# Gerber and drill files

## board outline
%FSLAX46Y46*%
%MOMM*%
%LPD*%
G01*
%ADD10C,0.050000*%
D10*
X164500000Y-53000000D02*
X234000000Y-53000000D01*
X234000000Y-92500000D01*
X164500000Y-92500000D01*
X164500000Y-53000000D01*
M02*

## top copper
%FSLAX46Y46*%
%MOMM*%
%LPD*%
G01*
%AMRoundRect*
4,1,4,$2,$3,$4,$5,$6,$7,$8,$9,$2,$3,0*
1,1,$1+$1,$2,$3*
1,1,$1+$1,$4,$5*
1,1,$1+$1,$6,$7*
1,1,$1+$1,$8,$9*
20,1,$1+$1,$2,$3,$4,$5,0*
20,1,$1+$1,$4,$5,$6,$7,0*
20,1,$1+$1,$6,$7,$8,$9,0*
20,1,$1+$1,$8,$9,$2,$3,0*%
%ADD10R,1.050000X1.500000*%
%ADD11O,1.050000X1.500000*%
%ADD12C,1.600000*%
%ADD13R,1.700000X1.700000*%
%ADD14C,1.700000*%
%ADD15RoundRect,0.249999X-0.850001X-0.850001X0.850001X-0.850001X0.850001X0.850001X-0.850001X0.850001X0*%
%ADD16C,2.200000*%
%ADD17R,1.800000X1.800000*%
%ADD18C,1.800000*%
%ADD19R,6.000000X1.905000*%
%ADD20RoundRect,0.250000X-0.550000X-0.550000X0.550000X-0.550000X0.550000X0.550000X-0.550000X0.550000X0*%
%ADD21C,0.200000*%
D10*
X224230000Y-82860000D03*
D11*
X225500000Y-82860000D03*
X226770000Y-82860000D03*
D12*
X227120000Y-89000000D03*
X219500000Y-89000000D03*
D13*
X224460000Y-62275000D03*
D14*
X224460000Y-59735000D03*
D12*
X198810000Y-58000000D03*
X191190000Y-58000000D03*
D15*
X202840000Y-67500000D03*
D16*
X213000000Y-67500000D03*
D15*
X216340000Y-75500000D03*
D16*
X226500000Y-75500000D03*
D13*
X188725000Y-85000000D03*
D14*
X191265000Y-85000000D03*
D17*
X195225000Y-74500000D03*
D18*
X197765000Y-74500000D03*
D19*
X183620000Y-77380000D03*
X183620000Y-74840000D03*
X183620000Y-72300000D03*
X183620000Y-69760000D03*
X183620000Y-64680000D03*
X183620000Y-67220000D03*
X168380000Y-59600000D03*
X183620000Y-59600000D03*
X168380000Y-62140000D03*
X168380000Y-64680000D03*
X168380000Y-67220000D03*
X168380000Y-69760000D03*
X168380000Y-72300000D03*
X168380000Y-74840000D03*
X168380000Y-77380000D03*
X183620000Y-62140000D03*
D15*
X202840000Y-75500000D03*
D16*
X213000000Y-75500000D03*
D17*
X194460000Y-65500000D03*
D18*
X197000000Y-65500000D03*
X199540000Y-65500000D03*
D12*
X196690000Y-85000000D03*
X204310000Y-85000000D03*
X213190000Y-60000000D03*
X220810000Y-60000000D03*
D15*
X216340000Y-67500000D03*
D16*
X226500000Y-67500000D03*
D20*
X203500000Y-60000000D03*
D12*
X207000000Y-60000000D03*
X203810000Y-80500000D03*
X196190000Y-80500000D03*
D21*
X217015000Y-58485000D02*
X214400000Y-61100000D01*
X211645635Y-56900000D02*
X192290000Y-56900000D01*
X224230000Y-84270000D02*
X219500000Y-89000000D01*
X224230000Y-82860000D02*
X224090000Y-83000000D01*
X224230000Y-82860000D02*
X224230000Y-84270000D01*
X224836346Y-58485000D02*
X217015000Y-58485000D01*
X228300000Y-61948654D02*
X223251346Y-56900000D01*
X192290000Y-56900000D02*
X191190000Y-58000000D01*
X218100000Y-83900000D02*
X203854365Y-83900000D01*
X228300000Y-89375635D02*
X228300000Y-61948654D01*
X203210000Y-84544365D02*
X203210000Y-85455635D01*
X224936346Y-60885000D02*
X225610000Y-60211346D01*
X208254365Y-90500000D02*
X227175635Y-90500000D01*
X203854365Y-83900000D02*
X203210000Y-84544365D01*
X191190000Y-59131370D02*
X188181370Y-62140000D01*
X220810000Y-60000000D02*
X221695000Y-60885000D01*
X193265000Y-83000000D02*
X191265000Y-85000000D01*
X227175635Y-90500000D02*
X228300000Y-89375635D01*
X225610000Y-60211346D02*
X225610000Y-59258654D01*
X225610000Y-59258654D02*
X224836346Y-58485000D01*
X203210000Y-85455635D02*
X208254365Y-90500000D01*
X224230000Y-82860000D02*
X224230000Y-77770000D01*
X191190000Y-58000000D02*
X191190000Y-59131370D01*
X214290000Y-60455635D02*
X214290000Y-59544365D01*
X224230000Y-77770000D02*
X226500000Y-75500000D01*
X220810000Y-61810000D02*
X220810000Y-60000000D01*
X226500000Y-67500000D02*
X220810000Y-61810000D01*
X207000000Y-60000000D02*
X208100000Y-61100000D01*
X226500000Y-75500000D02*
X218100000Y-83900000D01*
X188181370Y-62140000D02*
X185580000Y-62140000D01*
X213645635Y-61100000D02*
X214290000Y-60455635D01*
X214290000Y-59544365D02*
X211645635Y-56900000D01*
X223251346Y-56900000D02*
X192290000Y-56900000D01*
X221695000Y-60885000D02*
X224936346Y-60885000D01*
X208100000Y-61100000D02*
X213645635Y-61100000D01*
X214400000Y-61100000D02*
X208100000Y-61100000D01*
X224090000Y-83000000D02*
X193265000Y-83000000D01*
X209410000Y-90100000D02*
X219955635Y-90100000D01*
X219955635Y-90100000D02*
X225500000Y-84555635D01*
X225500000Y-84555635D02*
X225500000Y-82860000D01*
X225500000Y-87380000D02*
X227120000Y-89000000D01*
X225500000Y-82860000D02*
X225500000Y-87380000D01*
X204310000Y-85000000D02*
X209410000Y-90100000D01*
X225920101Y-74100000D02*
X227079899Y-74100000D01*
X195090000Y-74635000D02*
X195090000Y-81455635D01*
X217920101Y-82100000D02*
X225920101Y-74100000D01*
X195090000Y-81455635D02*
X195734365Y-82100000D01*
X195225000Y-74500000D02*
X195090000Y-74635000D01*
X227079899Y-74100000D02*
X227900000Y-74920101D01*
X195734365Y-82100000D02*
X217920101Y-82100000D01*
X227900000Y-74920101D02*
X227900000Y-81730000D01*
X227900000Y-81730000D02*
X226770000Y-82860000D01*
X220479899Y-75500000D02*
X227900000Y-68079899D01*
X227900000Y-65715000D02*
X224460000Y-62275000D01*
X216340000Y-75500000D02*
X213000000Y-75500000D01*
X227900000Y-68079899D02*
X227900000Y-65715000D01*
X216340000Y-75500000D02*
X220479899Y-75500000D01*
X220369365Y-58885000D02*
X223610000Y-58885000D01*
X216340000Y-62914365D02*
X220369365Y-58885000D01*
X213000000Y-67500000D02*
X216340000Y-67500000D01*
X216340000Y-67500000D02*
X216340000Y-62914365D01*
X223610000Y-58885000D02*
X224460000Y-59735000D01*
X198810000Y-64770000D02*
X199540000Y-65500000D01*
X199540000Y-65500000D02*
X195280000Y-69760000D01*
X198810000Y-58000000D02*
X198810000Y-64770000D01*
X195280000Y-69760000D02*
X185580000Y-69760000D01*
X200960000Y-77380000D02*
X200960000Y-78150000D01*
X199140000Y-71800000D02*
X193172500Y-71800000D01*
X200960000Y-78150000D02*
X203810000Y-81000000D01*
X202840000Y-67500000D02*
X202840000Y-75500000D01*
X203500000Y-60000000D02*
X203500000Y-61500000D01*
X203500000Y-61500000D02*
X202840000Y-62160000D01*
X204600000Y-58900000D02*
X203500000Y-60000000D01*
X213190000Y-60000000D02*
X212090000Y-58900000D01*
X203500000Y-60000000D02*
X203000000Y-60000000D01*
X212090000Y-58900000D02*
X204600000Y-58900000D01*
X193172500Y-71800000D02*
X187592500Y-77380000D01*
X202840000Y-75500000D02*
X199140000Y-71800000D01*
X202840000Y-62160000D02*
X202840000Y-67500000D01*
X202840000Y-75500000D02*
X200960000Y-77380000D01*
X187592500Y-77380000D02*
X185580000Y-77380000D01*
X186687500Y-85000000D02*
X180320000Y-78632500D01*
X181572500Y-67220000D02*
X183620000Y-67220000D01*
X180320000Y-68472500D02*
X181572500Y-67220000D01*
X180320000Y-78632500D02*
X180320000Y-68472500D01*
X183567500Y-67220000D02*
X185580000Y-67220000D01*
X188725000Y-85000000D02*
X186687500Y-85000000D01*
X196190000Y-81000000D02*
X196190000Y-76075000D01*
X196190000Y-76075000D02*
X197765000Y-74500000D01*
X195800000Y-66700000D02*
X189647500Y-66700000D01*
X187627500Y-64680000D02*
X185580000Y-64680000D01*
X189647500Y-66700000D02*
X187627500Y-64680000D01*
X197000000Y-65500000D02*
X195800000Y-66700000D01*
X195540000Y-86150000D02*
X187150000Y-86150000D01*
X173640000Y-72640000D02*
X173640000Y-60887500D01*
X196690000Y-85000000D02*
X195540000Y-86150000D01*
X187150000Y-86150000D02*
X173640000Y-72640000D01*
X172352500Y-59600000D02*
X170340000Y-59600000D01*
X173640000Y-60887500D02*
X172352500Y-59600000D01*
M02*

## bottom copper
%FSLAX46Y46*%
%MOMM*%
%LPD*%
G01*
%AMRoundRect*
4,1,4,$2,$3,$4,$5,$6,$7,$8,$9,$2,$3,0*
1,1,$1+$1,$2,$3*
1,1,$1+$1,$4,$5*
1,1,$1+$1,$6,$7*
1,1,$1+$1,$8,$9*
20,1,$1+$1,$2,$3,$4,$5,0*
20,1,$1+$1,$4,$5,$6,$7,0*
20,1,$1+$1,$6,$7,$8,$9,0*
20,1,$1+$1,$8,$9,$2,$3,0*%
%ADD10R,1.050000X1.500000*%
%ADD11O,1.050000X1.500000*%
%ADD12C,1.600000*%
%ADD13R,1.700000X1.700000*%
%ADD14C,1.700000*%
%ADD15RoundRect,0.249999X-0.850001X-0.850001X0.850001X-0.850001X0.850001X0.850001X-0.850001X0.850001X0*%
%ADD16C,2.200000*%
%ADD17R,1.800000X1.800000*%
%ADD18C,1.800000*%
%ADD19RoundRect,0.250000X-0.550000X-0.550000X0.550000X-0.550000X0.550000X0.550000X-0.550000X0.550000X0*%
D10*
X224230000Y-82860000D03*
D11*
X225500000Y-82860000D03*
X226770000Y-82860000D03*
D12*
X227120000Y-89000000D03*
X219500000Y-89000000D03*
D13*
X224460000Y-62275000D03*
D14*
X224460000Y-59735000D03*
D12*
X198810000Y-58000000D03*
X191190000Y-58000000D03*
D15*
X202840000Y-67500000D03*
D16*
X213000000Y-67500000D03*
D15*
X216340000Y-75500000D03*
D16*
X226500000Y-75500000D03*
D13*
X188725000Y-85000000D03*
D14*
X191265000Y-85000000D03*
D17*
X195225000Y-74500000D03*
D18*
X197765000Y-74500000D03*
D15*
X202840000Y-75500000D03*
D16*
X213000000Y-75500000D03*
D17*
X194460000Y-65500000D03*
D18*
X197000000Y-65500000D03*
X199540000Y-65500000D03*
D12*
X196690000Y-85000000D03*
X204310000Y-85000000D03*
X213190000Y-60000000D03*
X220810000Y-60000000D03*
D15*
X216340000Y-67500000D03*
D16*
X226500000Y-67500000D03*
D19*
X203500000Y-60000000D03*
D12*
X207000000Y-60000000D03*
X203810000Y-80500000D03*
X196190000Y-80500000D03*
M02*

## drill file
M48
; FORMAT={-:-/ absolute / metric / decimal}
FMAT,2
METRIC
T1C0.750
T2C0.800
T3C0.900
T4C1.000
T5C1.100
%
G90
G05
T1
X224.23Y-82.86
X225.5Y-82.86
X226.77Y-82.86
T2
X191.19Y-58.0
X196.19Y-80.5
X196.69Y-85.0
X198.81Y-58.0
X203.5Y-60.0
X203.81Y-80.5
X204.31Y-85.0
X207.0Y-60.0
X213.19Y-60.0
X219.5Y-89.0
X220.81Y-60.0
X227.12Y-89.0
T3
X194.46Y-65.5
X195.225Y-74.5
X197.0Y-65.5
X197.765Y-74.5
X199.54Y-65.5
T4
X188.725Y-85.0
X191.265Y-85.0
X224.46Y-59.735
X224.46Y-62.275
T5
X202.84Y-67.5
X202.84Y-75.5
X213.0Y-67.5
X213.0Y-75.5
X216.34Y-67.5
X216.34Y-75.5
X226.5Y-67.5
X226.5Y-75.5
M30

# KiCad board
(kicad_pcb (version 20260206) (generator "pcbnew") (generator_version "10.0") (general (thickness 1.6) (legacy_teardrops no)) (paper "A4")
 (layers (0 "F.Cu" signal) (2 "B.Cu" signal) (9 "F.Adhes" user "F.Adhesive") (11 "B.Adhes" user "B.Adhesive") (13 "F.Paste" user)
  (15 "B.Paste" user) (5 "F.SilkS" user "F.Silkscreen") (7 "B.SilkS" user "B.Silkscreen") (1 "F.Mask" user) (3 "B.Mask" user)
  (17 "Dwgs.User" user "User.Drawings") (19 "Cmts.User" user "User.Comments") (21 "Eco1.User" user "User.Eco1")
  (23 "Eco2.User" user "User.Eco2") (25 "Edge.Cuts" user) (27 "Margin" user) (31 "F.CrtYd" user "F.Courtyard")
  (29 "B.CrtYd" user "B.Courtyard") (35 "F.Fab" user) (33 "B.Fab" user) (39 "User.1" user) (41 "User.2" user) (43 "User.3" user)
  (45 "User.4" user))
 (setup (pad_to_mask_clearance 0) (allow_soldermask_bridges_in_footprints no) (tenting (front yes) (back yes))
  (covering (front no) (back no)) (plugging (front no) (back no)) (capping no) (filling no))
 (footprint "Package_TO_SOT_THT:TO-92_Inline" (layer "F.Cu") (at 224.23 82.86)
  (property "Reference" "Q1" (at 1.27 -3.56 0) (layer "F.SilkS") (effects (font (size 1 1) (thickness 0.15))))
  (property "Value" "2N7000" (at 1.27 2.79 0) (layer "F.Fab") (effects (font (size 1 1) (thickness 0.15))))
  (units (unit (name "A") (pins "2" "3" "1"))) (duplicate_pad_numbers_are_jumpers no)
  (pad "1" thru_hole rect (at 0 0) (size 1.05 1.5) (drill 0.75) (layers "*.Cu" "*.Mask") (remove_unused_layers no) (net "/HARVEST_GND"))
  (pad "2" thru_hole oval (at 1.27 0) (size 1.05 1.5) (drill 0.75) (layers "*.Cu" "*.Mask") (remove_unused_layers no) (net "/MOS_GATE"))
  (pad "3" thru_hole oval (at 2.54 0) (size 1.05 1.5) (drill 0.75) (layers "*.Cu" "*.Mask") (remove_unused_layers no) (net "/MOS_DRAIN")))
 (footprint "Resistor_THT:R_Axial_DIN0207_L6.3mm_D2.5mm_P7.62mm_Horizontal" (layer "F.Cu") (at 227.12 89 180)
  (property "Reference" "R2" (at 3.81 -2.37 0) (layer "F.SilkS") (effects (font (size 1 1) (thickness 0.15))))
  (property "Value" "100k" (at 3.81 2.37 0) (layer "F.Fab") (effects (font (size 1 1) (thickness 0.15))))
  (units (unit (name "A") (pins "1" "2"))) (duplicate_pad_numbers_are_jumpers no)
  (pad "1" thru_hole circle (at 0 0 180) (size 1.6 1.6) (drill 0.8) (layers "*.Cu" "*.Mask") (remove_unused_layers no) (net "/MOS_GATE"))
  (pad "2" thru_hole circle (at 7.62 0 180) (size 1.6 1.6) (drill 0.8) (layers "*.Cu" "*.Mask") (remove_unused_layers no)
   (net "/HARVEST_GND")))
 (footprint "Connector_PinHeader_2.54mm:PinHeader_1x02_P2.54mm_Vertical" (layer "F.Cu") (at 224.46 62.275 180)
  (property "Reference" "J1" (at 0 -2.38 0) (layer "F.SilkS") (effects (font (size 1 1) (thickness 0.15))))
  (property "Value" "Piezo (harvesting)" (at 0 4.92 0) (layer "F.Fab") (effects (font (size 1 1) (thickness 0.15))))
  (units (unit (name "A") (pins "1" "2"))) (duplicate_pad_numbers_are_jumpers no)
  (pad "1" thru_hole rect (at 0 0 180) (size 1.7 1.7) (drill 1) (layers "*.Cu" "*.Mask") (remove_unused_layers no) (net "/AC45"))
  (pad "2" thru_hole circle (at 0 2.54 180) (size 1.7 1.7) (drill 1) (layers "*.Cu" "*.Mask") (remove_unused_layers no) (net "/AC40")))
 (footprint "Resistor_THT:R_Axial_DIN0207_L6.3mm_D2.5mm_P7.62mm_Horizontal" (layer "F.Cu") (at 198.81 58 180)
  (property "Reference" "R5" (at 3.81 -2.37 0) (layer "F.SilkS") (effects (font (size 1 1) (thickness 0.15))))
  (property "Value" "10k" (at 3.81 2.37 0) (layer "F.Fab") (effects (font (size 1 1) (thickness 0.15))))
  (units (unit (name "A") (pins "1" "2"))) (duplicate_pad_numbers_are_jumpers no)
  (pad "1" thru_hole circle (at 0 0 180) (size 1.6 1.6) (drill 0.8) (layers "*.Cu" "*.Mask") (remove_unused_layers no) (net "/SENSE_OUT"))
  (pad "2" thru_hole circle (at 7.62 0 180) (size 1.6 1.6) (drill 0.8) (layers "*.Cu" "*.Mask") (remove_unused_layers no)
   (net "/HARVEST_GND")))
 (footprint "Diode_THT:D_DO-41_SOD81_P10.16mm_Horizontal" (layer "F.Cu") (at 202.84 67.5)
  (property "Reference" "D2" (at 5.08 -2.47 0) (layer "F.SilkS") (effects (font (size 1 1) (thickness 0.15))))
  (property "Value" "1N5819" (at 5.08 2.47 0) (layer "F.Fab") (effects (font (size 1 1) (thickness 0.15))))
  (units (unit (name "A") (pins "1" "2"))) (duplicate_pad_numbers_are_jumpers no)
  (pad "1" thru_hole roundrect (at 0 0) (size 2.2 2.2) (drill 1.1) (layers "*.Cu" "*.Mask") (remove_unused_layers no)
   (roundrect_rratio 0.113636) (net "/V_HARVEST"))
  (pad "2" thru_hole circle (at 10.16 0) (size 2.2 2.2) (drill 1.1) (layers "*.Cu" "*.Mask") (remove_unused_layers no) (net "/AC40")))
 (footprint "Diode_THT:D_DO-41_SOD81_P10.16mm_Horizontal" (layer "F.Cu") (at 216.34 75.5)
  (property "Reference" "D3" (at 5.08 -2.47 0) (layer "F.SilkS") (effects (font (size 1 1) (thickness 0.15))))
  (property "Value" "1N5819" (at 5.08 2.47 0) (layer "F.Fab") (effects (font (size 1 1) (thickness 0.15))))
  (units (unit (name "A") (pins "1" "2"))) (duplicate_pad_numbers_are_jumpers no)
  (pad "1" thru_hole roundrect (at 0 0) (size 2.2 2.2) (drill 1.1) (layers "*.Cu" "*.Mask") (remove_unused_layers no)
   (roundrect_rratio 0.113636) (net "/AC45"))
  (pad "2" thru_hole circle (at 10.16 0) (size 2.2 2.2) (drill 1.1) (layers "*.Cu" "*.Mask") (remove_unused_layers no) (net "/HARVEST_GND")))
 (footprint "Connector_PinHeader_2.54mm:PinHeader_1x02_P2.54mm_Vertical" (layer "F.Cu") (at 188.725 85 90)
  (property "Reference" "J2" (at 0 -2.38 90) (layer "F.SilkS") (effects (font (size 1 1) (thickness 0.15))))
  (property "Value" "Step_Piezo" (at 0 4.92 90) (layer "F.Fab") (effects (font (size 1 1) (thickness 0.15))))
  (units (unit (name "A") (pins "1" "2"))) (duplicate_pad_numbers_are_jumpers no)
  (pad "1" thru_hole rect (at 0 0 90) (size 1.7 1.7) (drill 1) (layers "*.Cu" "*.Mask") (remove_unused_layers no) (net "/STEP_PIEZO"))
  (pad "2" thru_hole circle (at 0 2.54 90) (size 1.7 1.7) (drill 1) (layers "*.Cu" "*.Mask") (remove_unused_layers no) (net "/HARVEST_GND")))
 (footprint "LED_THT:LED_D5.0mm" (layer "F.Cu") (at 195.225 74.5)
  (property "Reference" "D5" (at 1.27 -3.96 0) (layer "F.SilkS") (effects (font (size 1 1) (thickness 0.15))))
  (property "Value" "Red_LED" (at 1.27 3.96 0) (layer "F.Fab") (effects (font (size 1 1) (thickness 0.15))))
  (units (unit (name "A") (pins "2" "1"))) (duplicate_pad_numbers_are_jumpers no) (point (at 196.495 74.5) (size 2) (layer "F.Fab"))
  (pad "1" thru_hole rect (at 0 0) (size 1.8 1.8) (drill 0.9) (layers "*.Cu" "*.Mask") (remove_unused_layers no) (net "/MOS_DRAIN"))
  (pad "2" thru_hole circle (at 2.54 0) (size 1.8 1.8) (drill 0.9) (layers "*.Cu" "*.Mask") (remove_unused_layers no) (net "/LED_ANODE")))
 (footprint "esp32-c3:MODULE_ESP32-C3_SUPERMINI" (layer "F.Cu") (at 176 69.5)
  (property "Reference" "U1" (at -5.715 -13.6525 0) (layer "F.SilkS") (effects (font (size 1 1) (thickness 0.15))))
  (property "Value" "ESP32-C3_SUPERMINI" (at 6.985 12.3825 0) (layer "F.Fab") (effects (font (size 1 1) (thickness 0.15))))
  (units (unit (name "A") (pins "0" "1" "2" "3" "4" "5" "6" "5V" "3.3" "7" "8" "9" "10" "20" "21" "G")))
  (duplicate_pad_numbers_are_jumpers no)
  (pad "0" smd rect (at 7.62 7.88) (size 6 1.905) (layers "F.Cu" "F.Mask" "F.Paste") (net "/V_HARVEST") (solder_mask_margin 0.102))
  (pad "1" smd rect (at 7.62 5.34) (size 6 1.905) (layers "F.Cu" "F.Mask" "F.Paste") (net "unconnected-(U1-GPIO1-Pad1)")
   (solder_mask_margin 0.102))
  (pad "2" smd rect (at 7.62 2.8) (size 6 1.905) (layers "F.Cu" "F.Mask" "F.Paste") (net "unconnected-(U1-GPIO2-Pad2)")
   (solder_mask_margin 0.102))
  (pad "3" smd rect (at 7.62 0.26) (size 6 1.905) (layers "F.Cu" "F.Mask" "F.Paste") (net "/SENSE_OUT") (solder_mask_margin 0.102))
  (pad "3.3" smd rect (at 7.62 -4.82) (size 6 1.905) (layers "F.Cu" "F.Mask" "F.Paste") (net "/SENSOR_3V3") (solder_mask_margin 0.102))
  (pad "4" smd rect (at 7.62 -2.28) (size 6 1.905) (layers "F.Cu" "F.Mask" "F.Paste") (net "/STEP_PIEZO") (solder_mask_margin 0.102))
  (pad "5" smd rect (at -7.62 -9.9) (size 6 1.905) (layers "F.Cu" "F.Mask" "F.Paste") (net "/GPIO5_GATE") (solder_mask_margin 0.102))
  (pad "5V" smd rect (at 7.62 -9.9) (size 6 1.905) (layers "F.Cu" "F.Mask" "F.Paste") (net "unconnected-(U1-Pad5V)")
   (solder_mask_margin 0.102))
  (pad "6" smd rect (at -7.62 -7.36) (size 6 1.905) (layers "F.Cu" "F.Mask" "F.Paste") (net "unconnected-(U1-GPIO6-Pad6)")
   (solder_mask_margin 0.102))
  (pad "7" smd rect (at -7.62 -4.82) (size 6 1.905) (layers "F.Cu" "F.Mask" "F.Paste") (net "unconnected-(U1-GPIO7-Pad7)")
   (solder_mask_margin 0.102))
  (pad "8" smd rect (at -7.62 -2.28) (size 6 1.905) (layers "F.Cu" "F.Mask" "F.Paste") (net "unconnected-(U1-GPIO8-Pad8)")
   (solder_mask_margin 0.102))
  (pad "9" smd rect (at -7.62 0.26) (size 6 1.905) (layers "F.Cu" "F.Mask" "F.Paste") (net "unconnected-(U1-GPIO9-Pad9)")
   (solder_mask_margin 0.102))
  (pad "10" smd rect (at -7.62 2.8) (size 6 1.905) (layers "F.Cu" "F.Mask" "F.Paste") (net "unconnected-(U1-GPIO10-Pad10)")
   (solder_mask_margin 0.102))
  (pad "20" smd rect (at -7.62 5.34) (size 6 1.905) (layers "F.Cu" "F.Mask" "F.Paste") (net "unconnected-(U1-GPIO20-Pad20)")
   (solder_mask_margin 0.102))
  (pad "21" smd rect (at -7.62 7.88) (size 6 1.905) (layers "F.Cu" "F.Mask" "F.Paste") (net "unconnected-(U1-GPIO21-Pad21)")
   (solder_mask_margin 0.102))
  (pad "G" smd rect (at 7.62 -7.36) (size 6 1.905) (layers "F.Cu" "F.Mask" "F.Paste") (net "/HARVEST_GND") (solder_mask_margin 0.102)))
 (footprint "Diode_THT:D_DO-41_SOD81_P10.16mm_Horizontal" (layer "F.Cu") (at 202.84 75.5)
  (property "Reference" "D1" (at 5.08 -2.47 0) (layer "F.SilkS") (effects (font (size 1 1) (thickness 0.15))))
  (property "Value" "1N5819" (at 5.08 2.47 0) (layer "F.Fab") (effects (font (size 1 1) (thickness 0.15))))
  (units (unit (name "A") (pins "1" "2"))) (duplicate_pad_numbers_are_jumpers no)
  (pad "1" thru_hole roundrect (at 0 0) (size 2.2 2.2) (drill 1.1) (layers "*.Cu" "*.Mask") (remove_unused_layers no)
   (roundrect_rratio 0.113636) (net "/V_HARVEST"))
  (pad "2" thru_hole circle (at 10.16 0) (size 2.2 2.2) (drill 1.1) (layers "*.Cu" "*.Mask") (remove_unused_layers no) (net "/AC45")))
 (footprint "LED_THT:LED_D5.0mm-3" (layer "F.Cu") (at 194.46 65.5)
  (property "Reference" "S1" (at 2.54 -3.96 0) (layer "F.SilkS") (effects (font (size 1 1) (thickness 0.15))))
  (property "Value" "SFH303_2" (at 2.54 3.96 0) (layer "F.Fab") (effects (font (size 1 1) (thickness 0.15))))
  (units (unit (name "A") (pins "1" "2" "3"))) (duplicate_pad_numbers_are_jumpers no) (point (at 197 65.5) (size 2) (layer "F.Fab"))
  (pad "1" thru_hole rect (at 0 0) (size 1.8 1.8) (drill 0.9) (layers "*.Cu" "*.Mask") (remove_unused_layers no)
   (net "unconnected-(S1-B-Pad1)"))
  (pad "2" thru_hole circle (at 2.54 0) (size 1.8 1.8) (drill 0.9) (layers "*.Cu" "*.Mask") (remove_unused_layers no) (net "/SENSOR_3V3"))
  (pad "3" thru_hole circle (at 5.08 0) (size 1.8 1.8) (drill 0.9) (layers "*.Cu" "*.Mask") (remove_unused_layers no) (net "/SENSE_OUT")))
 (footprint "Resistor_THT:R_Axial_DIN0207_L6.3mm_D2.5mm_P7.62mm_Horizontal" (layer "F.Cu") (at 196.69 85)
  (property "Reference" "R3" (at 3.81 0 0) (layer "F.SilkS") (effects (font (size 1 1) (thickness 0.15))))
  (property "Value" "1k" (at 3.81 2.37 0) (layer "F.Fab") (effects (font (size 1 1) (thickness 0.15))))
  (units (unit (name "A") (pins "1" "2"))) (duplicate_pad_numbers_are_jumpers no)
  (pad "1" thru_hole circle (at 0 0) (size 1.6 1.6) (drill 0.8) (layers "*.Cu" "*.Mask") (remove_unused_layers no) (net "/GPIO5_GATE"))
  (pad "2" thru_hole circle (at 7.62 0) (size 1.6 1.6) (drill 0.8) (layers "*.Cu" "*.Mask") (remove_unused_layers no) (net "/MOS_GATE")))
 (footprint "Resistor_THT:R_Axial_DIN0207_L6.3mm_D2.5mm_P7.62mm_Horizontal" (layer "F.Cu") (at 213.19 60)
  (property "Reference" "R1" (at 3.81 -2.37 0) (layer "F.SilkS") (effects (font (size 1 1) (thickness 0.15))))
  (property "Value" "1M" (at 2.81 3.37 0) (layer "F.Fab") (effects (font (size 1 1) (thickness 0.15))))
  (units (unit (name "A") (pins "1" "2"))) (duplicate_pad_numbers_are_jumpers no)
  (pad "1" thru_hole circle (at 0 0) (size 1.6 1.6) (drill 0.8) (layers "*.Cu" "*.Mask") (remove_unused_layers no) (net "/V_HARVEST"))
  (pad "2" thru_hole circle (at 7.62 0) (size 1.6 1.6) (drill 0.8) (layers "*.Cu" "*.Mask") (remove_unused_layers no) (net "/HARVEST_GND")))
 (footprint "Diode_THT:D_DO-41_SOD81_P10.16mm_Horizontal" (layer "F.Cu") (at 216.34 67.5)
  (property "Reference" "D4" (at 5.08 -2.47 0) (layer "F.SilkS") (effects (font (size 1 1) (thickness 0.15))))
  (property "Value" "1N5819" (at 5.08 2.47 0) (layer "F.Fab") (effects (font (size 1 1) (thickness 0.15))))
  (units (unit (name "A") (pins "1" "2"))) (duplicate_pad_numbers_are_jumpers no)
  (pad "1" thru_hole roundrect (at 0 0) (size 2.2 2.2) (drill 1.1) (layers "*.Cu" "*.Mask") (remove_unused_layers no)
   (roundrect_rratio 0.113636) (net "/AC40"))
  (pad "2" thru_hole circle (at 10.16 0) (size 2.2 2.2) (drill 1.1) (layers "*.Cu" "*.Mask") (remove_unused_layers no) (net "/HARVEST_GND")))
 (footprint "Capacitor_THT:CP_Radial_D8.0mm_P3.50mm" (layer "F.Cu") (at 203.5 60)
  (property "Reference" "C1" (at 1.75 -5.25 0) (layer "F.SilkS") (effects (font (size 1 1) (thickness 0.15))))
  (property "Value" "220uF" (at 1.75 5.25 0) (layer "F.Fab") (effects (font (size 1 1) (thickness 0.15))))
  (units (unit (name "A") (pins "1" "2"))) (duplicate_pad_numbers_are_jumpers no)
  (pad "1" thru_hole roundrect (at 0 0) (size 1.6 1.6) (drill 0.8) (layers "*.Cu" "*.Mask") (remove_unused_layers no)
   (roundrect_rratio 0.15625) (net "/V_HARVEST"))
  (pad "2" thru_hole circle (at 3.5 0) (size 1.6 1.6) (drill 0.8) (layers "*.Cu" "*.Mask") (remove_unused_layers no) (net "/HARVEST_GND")))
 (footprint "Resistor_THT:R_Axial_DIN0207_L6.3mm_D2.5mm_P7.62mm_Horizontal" (layer "F.Cu") (at 203.81 80.5 180)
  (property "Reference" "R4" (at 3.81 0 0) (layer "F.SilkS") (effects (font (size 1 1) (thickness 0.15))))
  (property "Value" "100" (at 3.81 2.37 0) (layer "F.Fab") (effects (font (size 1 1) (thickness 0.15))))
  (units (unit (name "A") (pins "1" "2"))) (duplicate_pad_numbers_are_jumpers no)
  (pad "1" thru_hole circle (at 0 0 180) (size 1.6 1.6) (drill 0.8) (layers "*.Cu" "*.Mask") (remove_unused_layers no) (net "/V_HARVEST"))
  (pad "2" thru_hole circle (at 7.62 0 180) (size 1.6 1.6) (drill 0.8) (layers "*.Cu" "*.Mask") (remove_unused_layers no) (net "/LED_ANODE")))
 (gr_rect (start 164.5 53) (end 234 92.5) (stroke (width 0.05) (type solid)) (fill no) (layer "Edge.Cuts"))
 (segment (start 217.015 58.485) (end 214.4 61.1) (width 0.2) (layer "F.Cu") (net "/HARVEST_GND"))
 (segment (start 211.645635 56.9) (end 192.29 56.9) (width 0.2) (layer "F.Cu") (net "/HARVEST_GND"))
 (segment (start 224.23 84.27) (end 219.5 89) (width 0.2) (layer "F.Cu") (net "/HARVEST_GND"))
 (segment (start 224.23 82.86) (end 224.09 83) (width 0.2) (layer "F.Cu") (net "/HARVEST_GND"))
 (segment (start 224.23 82.86) (end 224.23 84.27) (width 0.2) (layer "F.Cu") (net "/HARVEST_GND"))
 (segment (start 224.836346 58.485) (end 217.015 58.485) (width 0.2) (layer "F.Cu") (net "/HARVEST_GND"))
 (segment (start 228.3 61.948654) (end 223.251346 56.9) (width 0.2) (layer "F.Cu") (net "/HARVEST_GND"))
 (segment (start 192.29 56.9) (end 191.19 58) (width 0.2) (layer "F.Cu") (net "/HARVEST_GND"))
 (segment (start 218.1 83.9) (end 203.854365 83.9) (width 0.2) (layer "F.Cu") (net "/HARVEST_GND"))
 (segment (start 228.3 89.375635) (end 228.3 61.948654) (width 0.2) (layer "F.Cu") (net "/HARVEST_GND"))
 (segment (start 203.21 84.544365) (end 203.21 85.455635) (width 0.2) (layer "F.Cu") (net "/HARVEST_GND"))
 (segment (start 224.936346 60.885) (end 225.61 60.211346) (width 0.2) (layer "F.Cu") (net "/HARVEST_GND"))
 (segment (start 208.254365 90.5) (end 227.175635 90.5) (width 0.2) (layer "F.Cu") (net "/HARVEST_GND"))
 (segment (start 203.854365 83.9) (end 203.21 84.544365) (width 0.2) (layer "F.Cu") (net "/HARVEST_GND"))
 (segment (start 191.19 59.13137) (end 188.18137 62.14) (width 0.2) (layer "F.Cu") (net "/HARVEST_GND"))
 (segment (start 220.81 60) (end 221.695 60.885) (width 0.2) (layer "F.Cu") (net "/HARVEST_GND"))
 (segment (start 193.265 83) (end 191.265 85) (width 0.2) (layer "F.Cu") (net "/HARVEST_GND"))
 (segment (start 227.175635 90.5) (end 228.3 89.375635) (width 0.2) (layer "F.Cu") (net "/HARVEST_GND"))
 (segment (start 225.61 60.211346) (end 225.61 59.258654) (width 0.2) (layer "F.Cu") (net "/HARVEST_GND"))
 (segment (start 225.61 59.258654) (end 224.836346 58.485) (width 0.2) (layer "F.Cu") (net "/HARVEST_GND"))
 (segment (start 203.21 85.455635) (end 208.254365 90.5) (width 0.2) (layer "F.Cu") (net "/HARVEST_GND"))
 (segment (start 224.23 82.86) (end 224.23 77.77) (width 0.2) (layer "F.Cu") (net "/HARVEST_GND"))
 (segment (start 191.19 58) (end 191.19 59.13137) (width 0.2) (layer "F.Cu") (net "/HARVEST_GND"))
 (segment (start 214.29 60.455635) (end 214.29 59.544365) (width 0.2) (layer "F.Cu") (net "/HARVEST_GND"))
 (segment (start 224.23 77.77) (end 226.5 75.5) (width 0.2) (layer "F.Cu") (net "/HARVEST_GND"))
 (segment (start 220.81 61.81) (end 220.81 60) (width 0.2) (layer "F.Cu") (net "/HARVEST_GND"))
 (segment (start 226.5 67.5) (end 220.81 61.81) (width 0.2) (layer "F.Cu") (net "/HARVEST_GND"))
 (segment (start 207 60) (end 208.1 61.1) (width 0.2) (layer "F.Cu") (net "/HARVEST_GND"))
 (segment (start 226.5 75.5) (end 218.1 83.9) (width 0.2) (layer "F.Cu") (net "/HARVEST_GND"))
 (segment (start 188.18137 62.14) (end 185.58 62.14) (width 0.2) (layer "F.Cu") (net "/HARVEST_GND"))
 (segment (start 213.645635 61.1) (end 214.29 60.455635) (width 0.2) (layer "F.Cu") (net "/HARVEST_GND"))
 (segment (start 214.29 59.544365) (end 211.645635 56.9) (width 0.2) (layer "F.Cu") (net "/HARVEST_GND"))
 (segment (start 223.251346 56.9) (end 192.29 56.9) (width 0.2) (layer "F.Cu") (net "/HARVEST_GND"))
 (segment (start 221.695 60.885) (end 224.936346 60.885) (width 0.2) (layer "F.Cu") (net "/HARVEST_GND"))
 (segment (start 208.1 61.1) (end 213.645635 61.1) (width 0.2) (layer "F.Cu") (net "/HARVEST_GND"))
 (segment (start 214.4 61.1) (end 208.1 61.1) (width 0.2) (layer "F.Cu") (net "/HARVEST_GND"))
 (segment (start 224.09 83) (end 193.265 83) (width 0.2) (layer "F.Cu") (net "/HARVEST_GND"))
 (segment (start 209.41 90.1) (end 219.955635 90.1) (width 0.2) (layer "F.Cu") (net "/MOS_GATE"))
 (segment (start 219.955635 90.1) (end 225.5 84.555635) (width 0.2) (layer "F.Cu") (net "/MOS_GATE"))
 (segment (start 225.5 84.555635) (end 225.5 82.86) (width 0.2) (layer "F.Cu") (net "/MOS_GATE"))
 (segment (start 225.5 87.38) (end 227.12 89) (width 0.2) (layer "F.Cu") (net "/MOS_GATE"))
 (segment (start 225.5 82.86) (end 225.5 87.38) (width 0.2) (layer "F.Cu") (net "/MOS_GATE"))
 (segment (start 204.31 85) (end 209.41 90.1) (width 0.2) (layer "F.Cu") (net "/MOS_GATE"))
 (segment (start 225.920101 74.1) (end 227.079899 74.1) (width 0.2) (layer "F.Cu") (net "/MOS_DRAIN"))
 (segment (start 195.09 74.635) (end 195.09 81.455635) (width 0.2) (layer "F.Cu") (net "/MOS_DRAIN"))
 (segment (start 217.920101 82.1) (end 225.920101 74.1) (width 0.2) (layer "F.Cu") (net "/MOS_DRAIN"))
 (segment (start 195.09 81.455635) (end 195.734365 82.1) (width 0.2) (layer "F.Cu") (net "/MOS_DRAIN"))
 (segment (start 195.225 74.5) (end 195.09 74.635) (width 0.2) (layer "F.Cu") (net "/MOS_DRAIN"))
 (segment (start 227.079899 74.1) (end 227.9 74.920101) (width 0.2) (layer "F.Cu") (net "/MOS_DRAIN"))
 (segment (start 195.734365 82.1) (end 217.920101 82.1) (width 0.2) (layer "F.Cu") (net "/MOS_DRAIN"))
 (segment (start 227.9 74.920101) (end 227.9 81.73) (width 0.2) (layer "F.Cu") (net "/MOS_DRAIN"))
 (segment (start 227.9 81.73) (end 226.77 82.86) (width 0.2) (layer "F.Cu") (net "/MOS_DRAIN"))
 (segment (start 220.479899 75.5) (end 227.9 68.079899) (width 0.2) (layer "F.Cu") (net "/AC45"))
 (segment (start 227.9 65.715) (end 224.46 62.275) (width 0.2) (layer "F.Cu") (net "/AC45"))
 (segment (start 216.34 75.5) (end 213 75.5) (width 0.2) (layer "F.Cu") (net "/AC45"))
 (segment (start 227.9 68.079899) (end 227.9 65.715) (width 0.2) (layer "F.Cu") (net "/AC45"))
 (segment (start 216.34 75.5) (end 220.479899 75.5) (width 0.2) (layer "F.Cu") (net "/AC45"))
 (segment (start 220.369365 58.885) (end 223.61 58.885) (width 0.2) (layer "F.Cu") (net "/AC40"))
 (segment (start 216.34 62.914365) (end 220.369365 58.885) (width 0.2) (layer "F.Cu") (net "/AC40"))
 (segment (start 213 67.5) (end 216.34 67.5) (width 0.2) (layer "F.Cu") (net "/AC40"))
 (segment (start 216.34 67.5) (end 216.34 62.914365) (width 0.2) (layer "F.Cu") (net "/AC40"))
 (segment (start 223.61 58.885) (end 224.46 59.735) (width 0.2) (layer "F.Cu") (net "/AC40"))
 (segment (start 198.81 64.77) (end 199.54 65.5) (width 0.2) (layer "F.Cu") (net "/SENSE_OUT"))
 (segment (start 199.54 65.5) (end 195.28 69.76) (width 0.2) (layer "F.Cu") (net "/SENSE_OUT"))
 (segment (start 198.81 58) (end 198.81 64.77) (width 0.2) (layer "F.Cu") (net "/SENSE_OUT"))
 (segment (start 195.28 69.76) (end 185.58 69.76) (width 0.2) (layer "F.Cu") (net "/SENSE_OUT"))
 (segment (start 200.96 77.38) (end 200.96 78.15) (width 0.2) (layer "F.Cu") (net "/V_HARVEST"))
 (segment (start 199.14 71.8) (end 193.1725 71.8) (width 0.2) (layer "F.Cu") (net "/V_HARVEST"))
 (segment (start 200.96 78.15) (end 203.81 81) (width 0.2) (layer "F.Cu") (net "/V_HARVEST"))
 (segment (start 202.84 67.5) (end 202.84 75.5) (width 0.2) (layer "F.Cu") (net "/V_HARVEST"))
 (segment (start 203.5 60) (end 203.5 61.5) (width 0.2) (layer "F.Cu") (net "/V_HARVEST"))
 (segment (start 203.5 61.5) (end 202.84 62.16) (width 0.2) (layer "F.Cu") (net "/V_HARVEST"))
 (segment (start 204.6 58.9) (end 203.5 60) (width 0.2) (layer "F.Cu") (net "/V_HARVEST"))
 (segment (start 213.19 60) (end 212.09 58.9) (width 0.2) (layer "F.Cu") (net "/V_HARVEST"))
 (segment (start 203.5 60) (end 203 60) (width 0.2) (layer "F.Cu") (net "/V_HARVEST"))
 (segment (start 212.09 58.9) (end 204.6 58.9) (width 0.2) (layer "F.Cu") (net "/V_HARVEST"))
 (segment (start 193.1725 71.8) (end 187.5925 77.38) (width 0.2) (layer "F.Cu") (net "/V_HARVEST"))
 (segment (start 202.84 75.5) (end 199.14 71.8) (width 0.2) (layer "F.Cu") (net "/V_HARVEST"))
 (segment (start 202.84 62.16) (end 202.84 67.5) (width 0.2) (layer "F.Cu") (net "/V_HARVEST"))
 (segment (start 202.84 75.5) (end 200.96 77.38) (width 0.2) (layer "F.Cu") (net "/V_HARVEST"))
 (segment (start 187.5925 77.38) (end 185.58 77.38) (width 0.2) (layer "F.Cu") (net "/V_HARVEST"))
 (segment (start 186.6875 85) (end 180.32 78.6325) (width 0.2) (layer "F.Cu") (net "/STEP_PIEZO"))
 (segment (start 181.5725 67.22) (end 183.62 67.22) (width 0.2) (layer "F.Cu") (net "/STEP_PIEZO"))
 (segment (start 180.32 68.4725) (end 181.5725 67.22) (width 0.2) (layer "F.Cu") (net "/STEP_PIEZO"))
 (segment (start 180.32 78.6325) (end 180.32 68.4725) (width 0.2) (layer "F.Cu") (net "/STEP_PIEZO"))
 (segment (start 183.5675 67.22) (end 185.58 67.22) (width 0.2) (layer "F.Cu") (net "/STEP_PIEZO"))
 (segment (start 188.725 85) (end 186.6875 85) (width 0.2) (layer "F.Cu") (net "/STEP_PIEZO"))
 (segment (start 196.19 81) (end 196.19 76.075) (width 0.2) (layer "F.Cu") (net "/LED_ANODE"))
 (segment (start 196.19 76.075) (end 197.765 74.5) (width 0.2) (layer "F.Cu") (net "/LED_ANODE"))
 (segment (start 195.8 66.7) (end 189.6475 66.7) (width 0.2) (layer "F.Cu") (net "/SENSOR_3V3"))
 (segment (start 187.6275 64.68) (end 185.58 64.68) (width 0.2) (layer "F.Cu") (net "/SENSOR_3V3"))
 (segment (start 189.6475 66.7) (end 187.6275 64.68) (width 0.2) (layer "F.Cu") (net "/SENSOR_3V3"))
 (segment (start 197 65.5) (end 195.8 66.7) (width 0.2) (layer "F.Cu") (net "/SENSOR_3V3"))
 (segment (start 195.54 86.15) (end 187.15 86.15) (width 0.2) (layer "F.Cu") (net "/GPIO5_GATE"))
 (segment (start 173.64 72.64) (end 173.64 60.8875) (width 0.2) (layer "F.Cu") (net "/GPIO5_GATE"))
 (segment (start 196.69 85) (end 195.54 86.15) (width 0.2) (layer "F.Cu") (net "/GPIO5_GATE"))
 (segment (start 187.15 86.15) (end 173.64 72.64) (width 0.2) (layer "F.Cu") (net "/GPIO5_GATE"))
 (segment (start 172.3525 59.6) (end 170.34 59.6) (width 0.2) (layer "F.Cu") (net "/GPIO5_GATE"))
 (segment (start 173.64 60.8875) (end 172.3525 59.6) (width 0.2) (layer "F.Cu") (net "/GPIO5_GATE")))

